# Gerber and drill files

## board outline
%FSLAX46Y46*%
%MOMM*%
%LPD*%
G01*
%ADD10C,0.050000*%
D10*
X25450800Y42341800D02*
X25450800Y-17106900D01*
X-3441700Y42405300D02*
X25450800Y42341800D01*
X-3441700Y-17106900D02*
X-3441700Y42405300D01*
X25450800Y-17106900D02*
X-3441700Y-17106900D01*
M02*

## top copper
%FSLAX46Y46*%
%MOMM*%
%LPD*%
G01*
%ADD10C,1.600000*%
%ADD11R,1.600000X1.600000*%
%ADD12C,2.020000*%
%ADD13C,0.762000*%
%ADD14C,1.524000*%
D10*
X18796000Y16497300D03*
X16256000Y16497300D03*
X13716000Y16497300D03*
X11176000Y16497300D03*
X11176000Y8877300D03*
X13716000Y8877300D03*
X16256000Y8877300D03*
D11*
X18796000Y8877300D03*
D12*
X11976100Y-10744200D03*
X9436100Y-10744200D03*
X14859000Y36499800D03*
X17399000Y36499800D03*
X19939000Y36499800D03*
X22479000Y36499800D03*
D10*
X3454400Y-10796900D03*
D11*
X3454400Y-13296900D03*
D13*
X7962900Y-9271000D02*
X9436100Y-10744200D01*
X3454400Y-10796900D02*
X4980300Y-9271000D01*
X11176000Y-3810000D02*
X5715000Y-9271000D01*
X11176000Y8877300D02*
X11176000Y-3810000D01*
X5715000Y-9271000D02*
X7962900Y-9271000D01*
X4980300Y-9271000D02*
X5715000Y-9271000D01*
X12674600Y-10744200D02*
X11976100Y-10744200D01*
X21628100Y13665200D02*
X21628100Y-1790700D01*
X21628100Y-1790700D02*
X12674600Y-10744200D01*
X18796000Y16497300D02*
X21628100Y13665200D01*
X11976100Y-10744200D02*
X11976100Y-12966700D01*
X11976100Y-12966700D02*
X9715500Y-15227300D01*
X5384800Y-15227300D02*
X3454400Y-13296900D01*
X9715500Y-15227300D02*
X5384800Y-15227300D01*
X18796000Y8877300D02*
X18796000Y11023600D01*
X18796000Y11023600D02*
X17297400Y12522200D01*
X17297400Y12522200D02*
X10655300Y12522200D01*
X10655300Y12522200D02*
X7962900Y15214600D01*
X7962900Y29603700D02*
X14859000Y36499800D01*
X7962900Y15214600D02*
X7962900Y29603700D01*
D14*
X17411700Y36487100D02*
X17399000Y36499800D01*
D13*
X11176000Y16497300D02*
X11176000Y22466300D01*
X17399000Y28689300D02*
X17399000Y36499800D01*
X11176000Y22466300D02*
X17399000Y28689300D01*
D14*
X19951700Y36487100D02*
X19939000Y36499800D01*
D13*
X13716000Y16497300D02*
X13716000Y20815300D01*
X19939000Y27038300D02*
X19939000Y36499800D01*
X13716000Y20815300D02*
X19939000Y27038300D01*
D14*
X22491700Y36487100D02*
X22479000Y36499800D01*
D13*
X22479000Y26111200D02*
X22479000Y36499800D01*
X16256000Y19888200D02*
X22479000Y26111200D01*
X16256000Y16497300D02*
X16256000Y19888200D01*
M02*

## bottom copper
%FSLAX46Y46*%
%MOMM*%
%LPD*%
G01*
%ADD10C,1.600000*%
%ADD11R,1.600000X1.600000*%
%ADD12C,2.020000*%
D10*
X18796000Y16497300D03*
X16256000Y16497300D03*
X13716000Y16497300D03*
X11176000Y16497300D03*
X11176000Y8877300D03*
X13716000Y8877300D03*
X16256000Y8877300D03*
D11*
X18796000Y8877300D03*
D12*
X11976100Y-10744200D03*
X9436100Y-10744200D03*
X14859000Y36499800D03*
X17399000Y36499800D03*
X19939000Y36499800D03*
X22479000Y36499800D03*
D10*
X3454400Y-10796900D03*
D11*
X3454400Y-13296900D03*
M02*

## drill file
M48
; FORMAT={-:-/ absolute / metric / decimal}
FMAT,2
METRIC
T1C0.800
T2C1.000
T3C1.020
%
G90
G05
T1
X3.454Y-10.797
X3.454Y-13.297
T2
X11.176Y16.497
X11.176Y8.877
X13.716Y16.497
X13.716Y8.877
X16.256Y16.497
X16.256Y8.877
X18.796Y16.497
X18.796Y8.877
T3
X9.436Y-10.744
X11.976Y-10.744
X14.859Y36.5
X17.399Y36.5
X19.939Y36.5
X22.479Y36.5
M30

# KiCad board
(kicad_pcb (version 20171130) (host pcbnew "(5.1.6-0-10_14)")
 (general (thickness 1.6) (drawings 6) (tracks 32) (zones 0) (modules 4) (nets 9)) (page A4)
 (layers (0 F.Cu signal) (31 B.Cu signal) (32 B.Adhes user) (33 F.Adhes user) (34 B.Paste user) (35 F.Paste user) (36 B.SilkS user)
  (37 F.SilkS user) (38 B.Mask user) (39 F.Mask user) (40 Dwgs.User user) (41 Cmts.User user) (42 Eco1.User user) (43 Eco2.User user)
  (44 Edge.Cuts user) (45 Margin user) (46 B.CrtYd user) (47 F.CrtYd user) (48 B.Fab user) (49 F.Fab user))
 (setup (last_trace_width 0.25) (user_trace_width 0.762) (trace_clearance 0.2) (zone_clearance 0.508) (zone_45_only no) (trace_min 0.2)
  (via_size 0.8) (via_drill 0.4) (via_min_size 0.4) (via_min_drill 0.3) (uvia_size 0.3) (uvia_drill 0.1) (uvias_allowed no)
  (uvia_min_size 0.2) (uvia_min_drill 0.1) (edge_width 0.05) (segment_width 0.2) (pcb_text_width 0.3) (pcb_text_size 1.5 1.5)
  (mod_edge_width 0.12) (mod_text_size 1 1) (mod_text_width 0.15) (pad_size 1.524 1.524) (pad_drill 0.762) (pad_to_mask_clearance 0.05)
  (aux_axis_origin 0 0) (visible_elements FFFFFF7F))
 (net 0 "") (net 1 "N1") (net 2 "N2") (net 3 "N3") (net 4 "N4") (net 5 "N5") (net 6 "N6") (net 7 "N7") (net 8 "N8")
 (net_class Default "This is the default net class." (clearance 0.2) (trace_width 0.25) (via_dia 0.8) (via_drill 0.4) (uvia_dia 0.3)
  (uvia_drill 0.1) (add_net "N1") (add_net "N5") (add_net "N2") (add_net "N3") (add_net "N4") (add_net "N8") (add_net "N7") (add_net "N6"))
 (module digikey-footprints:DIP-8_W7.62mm (layer B.Cu) (at 18.796 -8.8773 90)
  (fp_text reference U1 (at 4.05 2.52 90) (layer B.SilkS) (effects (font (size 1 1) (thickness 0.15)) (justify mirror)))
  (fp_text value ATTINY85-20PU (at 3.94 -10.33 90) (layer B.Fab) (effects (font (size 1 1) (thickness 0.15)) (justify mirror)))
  (pad 8 thru_hole circle (at 7.62 0 90) (size 1.6 1.6) (drill 1) (layers *.Cu *.Mask) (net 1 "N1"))
  (pad 7 thru_hole circle (at 7.62 -2.54 90) (size 1.6 1.6) (drill 1) (layers *.Cu *.Mask) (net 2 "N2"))
  (pad 6 thru_hole circle (at 7.62 -5.08 90) (size 1.6 1.6) (drill 1) (layers *.Cu *.Mask) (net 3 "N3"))
  (pad 5 thru_hole circle (at 7.62 -7.62 90) (size 1.6 1.6) (drill 1) (layers *.Cu *.Mask) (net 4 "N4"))
  (pad 4 thru_hole circle (at 0 -7.62 90) (size 1.6 1.6) (drill 1) (layers *.Cu *.Mask) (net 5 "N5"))
  (pad 3 thru_hole circle (at 0 -5.08 90) (size 1.6 1.6) (drill 1) (layers *.Cu *.Mask) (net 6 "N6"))
  (pad 2 thru_hole circle (at 0 -2.54 90) (size 1.6 1.6) (drill 1) (layers *.Cu *.Mask) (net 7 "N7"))
  (pad 1 thru_hole rect (at 0 0 90) (size 1.6 1.6) (drill 1) (layers *.Cu *.Mask) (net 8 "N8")))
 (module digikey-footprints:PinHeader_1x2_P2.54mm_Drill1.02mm (layer F.Cu) (at 9.4361 10.7442)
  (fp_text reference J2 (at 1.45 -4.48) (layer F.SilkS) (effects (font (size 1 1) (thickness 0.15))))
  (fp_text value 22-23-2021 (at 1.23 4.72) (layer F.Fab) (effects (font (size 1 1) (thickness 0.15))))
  (pad 2 thru_hole circle (at 2.54 0) (size 2.02 2.02) (drill 1.02) (layers *.Cu *.Mask) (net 1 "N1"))
  (pad 1 thru_hole circle (at 0 0) (size 2.02 2.02) (drill 1.02) (layers *.Cu *.Mask) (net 5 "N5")))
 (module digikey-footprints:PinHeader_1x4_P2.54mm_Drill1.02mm (layer F.Cu) (at 22.479 -36.4998 180)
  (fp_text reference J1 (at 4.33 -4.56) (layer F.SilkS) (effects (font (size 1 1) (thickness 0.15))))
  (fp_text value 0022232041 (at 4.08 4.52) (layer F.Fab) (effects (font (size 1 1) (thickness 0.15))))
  (pad 4 thru_hole circle (at 7.62 0 180) (size 2.02 2.02) (drill 1.02) (layers *.Cu *.Mask) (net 8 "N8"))
  (pad 3 thru_hole circle (at 5.08 0 180) (size 2.02 2.02) (drill 1.02) (layers *.Cu *.Mask) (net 4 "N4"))
  (pad 2 thru_hole circle (at 2.54 0 180) (size 2.02 2.02) (drill 1.02) (layers *.Cu *.Mask) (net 3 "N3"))
  (pad 1 thru_hole circle (at 0 0 180) (size 2.02 2.02) (drill 1.02) (layers *.Cu *.Mask) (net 2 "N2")))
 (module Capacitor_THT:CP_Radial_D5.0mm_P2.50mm (layer F.Cu) (at 3.4544 13.2969 90)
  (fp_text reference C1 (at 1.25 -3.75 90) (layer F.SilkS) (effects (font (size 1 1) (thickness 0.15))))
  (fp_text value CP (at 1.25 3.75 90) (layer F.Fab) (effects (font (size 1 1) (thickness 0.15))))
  (pad 2 thru_hole circle (at 2.5 0 90) (size 1.6 1.6) (drill 0.8) (layers *.Cu *.Mask) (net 5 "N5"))
  (pad 1 thru_hole rect (at 0 0 90) (size 1.6 1.6) (drill 0.8) (layers *.Cu *.Mask) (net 1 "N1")))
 (gr_line (start 25.4508 -42.3418) (end 25.4508 17.1069) (layer Edge.Cuts) (width 0.05))
 (gr_line (start -3.4417 -42.4053) (end 25.4508 -42.3418) (layer Edge.Cuts) (width 0.05))
 (gr_line (start -3.4417 17.1069) (end -3.4417 -42.4053) (layer Edge.Cuts) (width 0.05))
 (gr_line (start 25.4508 17.1069) (end -3.4417 17.1069) (layer Edge.Cuts) (width 0.05))
 (segment (start 7.9629 9.271) (end 9.4361 10.7442) (width 0.762) (layer F.Cu) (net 5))
 (segment (start 3.4544 10.7969) (end 4.9803 9.271) (width 0.762) (layer F.Cu) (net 5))
 (segment (start 11.176 3.81) (end 5.715 9.271) (width 0.762) (layer F.Cu) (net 5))
 (segment (start 11.176 -8.8773) (end 11.176 3.81) (width 0.762) (layer F.Cu) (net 5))
 (segment (start 5.715 9.271) (end 7.9629 9.271) (width 0.762) (layer F.Cu) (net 5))
 (segment (start 4.9803 9.271) (end 5.715 9.271) (width 0.762) (layer F.Cu) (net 5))
 (segment (start 12.6746 10.7442) (end 11.9761 10.7442) (width 0.762) (layer F.Cu) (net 1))
 (segment (start 21.6281 -13.6652) (end 21.6281 1.7907) (width 0.762) (layer F.Cu) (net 1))
 (segment (start 21.6281 1.7907) (end 12.6746 10.7442) (width 0.762) (layer F.Cu) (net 1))
 (segment (start 18.796 -16.4973) (end 21.6281 -13.6652) (width 0.762) (layer F.Cu) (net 1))
 (segment (start 11.9761 10.7442) (end 11.9761 12.9667) (width 0.762) (layer F.Cu) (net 1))
 (segment (start 11.9761 12.9667) (end 9.7155 15.2273) (width 0.762) (layer F.Cu) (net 1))
 (segment (start 5.3848 15.2273) (end 3.4544 13.2969) (width 0.762) (layer F.Cu) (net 1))
 (segment (start 9.7155 15.2273) (end 5.3848 15.2273) (width 0.762) (layer F.Cu) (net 1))
 (segment (start 18.796 -8.8773) (end 18.796 -11.0236) (width 0.762) (layer F.Cu) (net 8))
 (segment (start 18.796 -11.0236) (end 17.2974 -12.5222) (width 0.762) (layer F.Cu) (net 8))
 (segment (start 17.2974 -12.5222) (end 10.6553 -12.5222) (width 0.762) (layer F.Cu) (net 8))
 (segment (start 10.6553 -12.5222) (end 7.9629 -15.2146) (width 0.762) (layer F.Cu) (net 8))
 (segment (start 7.9629 -29.6037) (end 14.859 -36.4998) (width 0.762) (layer F.Cu) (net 8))
 (segment (start 7.9629 -15.2146) (end 7.9629 -29.6037) (width 0.762) (layer F.Cu) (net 8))
 (segment (start 17.4117 -36.4871) (end 17.399 -36.4998) (width 1.524) (layer F.Cu) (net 4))
 (segment (start 11.176 -16.4973) (end 11.176 -22.4663) (width 0.762) (layer F.Cu) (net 4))
 (segment (start 17.399 -28.6893) (end 17.399 -36.4998) (width 0.762) (layer F.Cu) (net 4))
 (segment (start 11.176 -22.4663) (end 17.399 -28.6893) (width 0.762) (layer F.Cu) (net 4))
 (segment (start 19.9517 -36.4871) (end 19.939 -36.4998) (width 1.524) (layer F.Cu) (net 3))
 (segment (start 13.716 -16.4973) (end 13.716 -20.8153) (width 0.762) (layer F.Cu) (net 3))
 (segment (start 19.939 -27.0383) (end 19.939 -36.4998) (width 0.762) (layer F.Cu) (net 3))
 (segment (start 13.716 -20.8153) (end 19.939 -27.0383) (width 0.762) (layer F.Cu) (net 3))
 (segment (start 22.4917 -36.4871) (end 22.479 -36.4998) (width 1.524) (layer F.Cu) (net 2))
 (segment (start 22.479 -26.1112) (end 22.479 -36.4998) (width 0.762) (layer F.Cu) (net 2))
 (segment (start 16.256 -19.8882) (end 22.479 -26.1112) (width 0.762) (layer F.Cu) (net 2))
 (segment (start 16.256 -16.4973) (end 16.256 -19.8882) (width 0.762) (layer F.Cu) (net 2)))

